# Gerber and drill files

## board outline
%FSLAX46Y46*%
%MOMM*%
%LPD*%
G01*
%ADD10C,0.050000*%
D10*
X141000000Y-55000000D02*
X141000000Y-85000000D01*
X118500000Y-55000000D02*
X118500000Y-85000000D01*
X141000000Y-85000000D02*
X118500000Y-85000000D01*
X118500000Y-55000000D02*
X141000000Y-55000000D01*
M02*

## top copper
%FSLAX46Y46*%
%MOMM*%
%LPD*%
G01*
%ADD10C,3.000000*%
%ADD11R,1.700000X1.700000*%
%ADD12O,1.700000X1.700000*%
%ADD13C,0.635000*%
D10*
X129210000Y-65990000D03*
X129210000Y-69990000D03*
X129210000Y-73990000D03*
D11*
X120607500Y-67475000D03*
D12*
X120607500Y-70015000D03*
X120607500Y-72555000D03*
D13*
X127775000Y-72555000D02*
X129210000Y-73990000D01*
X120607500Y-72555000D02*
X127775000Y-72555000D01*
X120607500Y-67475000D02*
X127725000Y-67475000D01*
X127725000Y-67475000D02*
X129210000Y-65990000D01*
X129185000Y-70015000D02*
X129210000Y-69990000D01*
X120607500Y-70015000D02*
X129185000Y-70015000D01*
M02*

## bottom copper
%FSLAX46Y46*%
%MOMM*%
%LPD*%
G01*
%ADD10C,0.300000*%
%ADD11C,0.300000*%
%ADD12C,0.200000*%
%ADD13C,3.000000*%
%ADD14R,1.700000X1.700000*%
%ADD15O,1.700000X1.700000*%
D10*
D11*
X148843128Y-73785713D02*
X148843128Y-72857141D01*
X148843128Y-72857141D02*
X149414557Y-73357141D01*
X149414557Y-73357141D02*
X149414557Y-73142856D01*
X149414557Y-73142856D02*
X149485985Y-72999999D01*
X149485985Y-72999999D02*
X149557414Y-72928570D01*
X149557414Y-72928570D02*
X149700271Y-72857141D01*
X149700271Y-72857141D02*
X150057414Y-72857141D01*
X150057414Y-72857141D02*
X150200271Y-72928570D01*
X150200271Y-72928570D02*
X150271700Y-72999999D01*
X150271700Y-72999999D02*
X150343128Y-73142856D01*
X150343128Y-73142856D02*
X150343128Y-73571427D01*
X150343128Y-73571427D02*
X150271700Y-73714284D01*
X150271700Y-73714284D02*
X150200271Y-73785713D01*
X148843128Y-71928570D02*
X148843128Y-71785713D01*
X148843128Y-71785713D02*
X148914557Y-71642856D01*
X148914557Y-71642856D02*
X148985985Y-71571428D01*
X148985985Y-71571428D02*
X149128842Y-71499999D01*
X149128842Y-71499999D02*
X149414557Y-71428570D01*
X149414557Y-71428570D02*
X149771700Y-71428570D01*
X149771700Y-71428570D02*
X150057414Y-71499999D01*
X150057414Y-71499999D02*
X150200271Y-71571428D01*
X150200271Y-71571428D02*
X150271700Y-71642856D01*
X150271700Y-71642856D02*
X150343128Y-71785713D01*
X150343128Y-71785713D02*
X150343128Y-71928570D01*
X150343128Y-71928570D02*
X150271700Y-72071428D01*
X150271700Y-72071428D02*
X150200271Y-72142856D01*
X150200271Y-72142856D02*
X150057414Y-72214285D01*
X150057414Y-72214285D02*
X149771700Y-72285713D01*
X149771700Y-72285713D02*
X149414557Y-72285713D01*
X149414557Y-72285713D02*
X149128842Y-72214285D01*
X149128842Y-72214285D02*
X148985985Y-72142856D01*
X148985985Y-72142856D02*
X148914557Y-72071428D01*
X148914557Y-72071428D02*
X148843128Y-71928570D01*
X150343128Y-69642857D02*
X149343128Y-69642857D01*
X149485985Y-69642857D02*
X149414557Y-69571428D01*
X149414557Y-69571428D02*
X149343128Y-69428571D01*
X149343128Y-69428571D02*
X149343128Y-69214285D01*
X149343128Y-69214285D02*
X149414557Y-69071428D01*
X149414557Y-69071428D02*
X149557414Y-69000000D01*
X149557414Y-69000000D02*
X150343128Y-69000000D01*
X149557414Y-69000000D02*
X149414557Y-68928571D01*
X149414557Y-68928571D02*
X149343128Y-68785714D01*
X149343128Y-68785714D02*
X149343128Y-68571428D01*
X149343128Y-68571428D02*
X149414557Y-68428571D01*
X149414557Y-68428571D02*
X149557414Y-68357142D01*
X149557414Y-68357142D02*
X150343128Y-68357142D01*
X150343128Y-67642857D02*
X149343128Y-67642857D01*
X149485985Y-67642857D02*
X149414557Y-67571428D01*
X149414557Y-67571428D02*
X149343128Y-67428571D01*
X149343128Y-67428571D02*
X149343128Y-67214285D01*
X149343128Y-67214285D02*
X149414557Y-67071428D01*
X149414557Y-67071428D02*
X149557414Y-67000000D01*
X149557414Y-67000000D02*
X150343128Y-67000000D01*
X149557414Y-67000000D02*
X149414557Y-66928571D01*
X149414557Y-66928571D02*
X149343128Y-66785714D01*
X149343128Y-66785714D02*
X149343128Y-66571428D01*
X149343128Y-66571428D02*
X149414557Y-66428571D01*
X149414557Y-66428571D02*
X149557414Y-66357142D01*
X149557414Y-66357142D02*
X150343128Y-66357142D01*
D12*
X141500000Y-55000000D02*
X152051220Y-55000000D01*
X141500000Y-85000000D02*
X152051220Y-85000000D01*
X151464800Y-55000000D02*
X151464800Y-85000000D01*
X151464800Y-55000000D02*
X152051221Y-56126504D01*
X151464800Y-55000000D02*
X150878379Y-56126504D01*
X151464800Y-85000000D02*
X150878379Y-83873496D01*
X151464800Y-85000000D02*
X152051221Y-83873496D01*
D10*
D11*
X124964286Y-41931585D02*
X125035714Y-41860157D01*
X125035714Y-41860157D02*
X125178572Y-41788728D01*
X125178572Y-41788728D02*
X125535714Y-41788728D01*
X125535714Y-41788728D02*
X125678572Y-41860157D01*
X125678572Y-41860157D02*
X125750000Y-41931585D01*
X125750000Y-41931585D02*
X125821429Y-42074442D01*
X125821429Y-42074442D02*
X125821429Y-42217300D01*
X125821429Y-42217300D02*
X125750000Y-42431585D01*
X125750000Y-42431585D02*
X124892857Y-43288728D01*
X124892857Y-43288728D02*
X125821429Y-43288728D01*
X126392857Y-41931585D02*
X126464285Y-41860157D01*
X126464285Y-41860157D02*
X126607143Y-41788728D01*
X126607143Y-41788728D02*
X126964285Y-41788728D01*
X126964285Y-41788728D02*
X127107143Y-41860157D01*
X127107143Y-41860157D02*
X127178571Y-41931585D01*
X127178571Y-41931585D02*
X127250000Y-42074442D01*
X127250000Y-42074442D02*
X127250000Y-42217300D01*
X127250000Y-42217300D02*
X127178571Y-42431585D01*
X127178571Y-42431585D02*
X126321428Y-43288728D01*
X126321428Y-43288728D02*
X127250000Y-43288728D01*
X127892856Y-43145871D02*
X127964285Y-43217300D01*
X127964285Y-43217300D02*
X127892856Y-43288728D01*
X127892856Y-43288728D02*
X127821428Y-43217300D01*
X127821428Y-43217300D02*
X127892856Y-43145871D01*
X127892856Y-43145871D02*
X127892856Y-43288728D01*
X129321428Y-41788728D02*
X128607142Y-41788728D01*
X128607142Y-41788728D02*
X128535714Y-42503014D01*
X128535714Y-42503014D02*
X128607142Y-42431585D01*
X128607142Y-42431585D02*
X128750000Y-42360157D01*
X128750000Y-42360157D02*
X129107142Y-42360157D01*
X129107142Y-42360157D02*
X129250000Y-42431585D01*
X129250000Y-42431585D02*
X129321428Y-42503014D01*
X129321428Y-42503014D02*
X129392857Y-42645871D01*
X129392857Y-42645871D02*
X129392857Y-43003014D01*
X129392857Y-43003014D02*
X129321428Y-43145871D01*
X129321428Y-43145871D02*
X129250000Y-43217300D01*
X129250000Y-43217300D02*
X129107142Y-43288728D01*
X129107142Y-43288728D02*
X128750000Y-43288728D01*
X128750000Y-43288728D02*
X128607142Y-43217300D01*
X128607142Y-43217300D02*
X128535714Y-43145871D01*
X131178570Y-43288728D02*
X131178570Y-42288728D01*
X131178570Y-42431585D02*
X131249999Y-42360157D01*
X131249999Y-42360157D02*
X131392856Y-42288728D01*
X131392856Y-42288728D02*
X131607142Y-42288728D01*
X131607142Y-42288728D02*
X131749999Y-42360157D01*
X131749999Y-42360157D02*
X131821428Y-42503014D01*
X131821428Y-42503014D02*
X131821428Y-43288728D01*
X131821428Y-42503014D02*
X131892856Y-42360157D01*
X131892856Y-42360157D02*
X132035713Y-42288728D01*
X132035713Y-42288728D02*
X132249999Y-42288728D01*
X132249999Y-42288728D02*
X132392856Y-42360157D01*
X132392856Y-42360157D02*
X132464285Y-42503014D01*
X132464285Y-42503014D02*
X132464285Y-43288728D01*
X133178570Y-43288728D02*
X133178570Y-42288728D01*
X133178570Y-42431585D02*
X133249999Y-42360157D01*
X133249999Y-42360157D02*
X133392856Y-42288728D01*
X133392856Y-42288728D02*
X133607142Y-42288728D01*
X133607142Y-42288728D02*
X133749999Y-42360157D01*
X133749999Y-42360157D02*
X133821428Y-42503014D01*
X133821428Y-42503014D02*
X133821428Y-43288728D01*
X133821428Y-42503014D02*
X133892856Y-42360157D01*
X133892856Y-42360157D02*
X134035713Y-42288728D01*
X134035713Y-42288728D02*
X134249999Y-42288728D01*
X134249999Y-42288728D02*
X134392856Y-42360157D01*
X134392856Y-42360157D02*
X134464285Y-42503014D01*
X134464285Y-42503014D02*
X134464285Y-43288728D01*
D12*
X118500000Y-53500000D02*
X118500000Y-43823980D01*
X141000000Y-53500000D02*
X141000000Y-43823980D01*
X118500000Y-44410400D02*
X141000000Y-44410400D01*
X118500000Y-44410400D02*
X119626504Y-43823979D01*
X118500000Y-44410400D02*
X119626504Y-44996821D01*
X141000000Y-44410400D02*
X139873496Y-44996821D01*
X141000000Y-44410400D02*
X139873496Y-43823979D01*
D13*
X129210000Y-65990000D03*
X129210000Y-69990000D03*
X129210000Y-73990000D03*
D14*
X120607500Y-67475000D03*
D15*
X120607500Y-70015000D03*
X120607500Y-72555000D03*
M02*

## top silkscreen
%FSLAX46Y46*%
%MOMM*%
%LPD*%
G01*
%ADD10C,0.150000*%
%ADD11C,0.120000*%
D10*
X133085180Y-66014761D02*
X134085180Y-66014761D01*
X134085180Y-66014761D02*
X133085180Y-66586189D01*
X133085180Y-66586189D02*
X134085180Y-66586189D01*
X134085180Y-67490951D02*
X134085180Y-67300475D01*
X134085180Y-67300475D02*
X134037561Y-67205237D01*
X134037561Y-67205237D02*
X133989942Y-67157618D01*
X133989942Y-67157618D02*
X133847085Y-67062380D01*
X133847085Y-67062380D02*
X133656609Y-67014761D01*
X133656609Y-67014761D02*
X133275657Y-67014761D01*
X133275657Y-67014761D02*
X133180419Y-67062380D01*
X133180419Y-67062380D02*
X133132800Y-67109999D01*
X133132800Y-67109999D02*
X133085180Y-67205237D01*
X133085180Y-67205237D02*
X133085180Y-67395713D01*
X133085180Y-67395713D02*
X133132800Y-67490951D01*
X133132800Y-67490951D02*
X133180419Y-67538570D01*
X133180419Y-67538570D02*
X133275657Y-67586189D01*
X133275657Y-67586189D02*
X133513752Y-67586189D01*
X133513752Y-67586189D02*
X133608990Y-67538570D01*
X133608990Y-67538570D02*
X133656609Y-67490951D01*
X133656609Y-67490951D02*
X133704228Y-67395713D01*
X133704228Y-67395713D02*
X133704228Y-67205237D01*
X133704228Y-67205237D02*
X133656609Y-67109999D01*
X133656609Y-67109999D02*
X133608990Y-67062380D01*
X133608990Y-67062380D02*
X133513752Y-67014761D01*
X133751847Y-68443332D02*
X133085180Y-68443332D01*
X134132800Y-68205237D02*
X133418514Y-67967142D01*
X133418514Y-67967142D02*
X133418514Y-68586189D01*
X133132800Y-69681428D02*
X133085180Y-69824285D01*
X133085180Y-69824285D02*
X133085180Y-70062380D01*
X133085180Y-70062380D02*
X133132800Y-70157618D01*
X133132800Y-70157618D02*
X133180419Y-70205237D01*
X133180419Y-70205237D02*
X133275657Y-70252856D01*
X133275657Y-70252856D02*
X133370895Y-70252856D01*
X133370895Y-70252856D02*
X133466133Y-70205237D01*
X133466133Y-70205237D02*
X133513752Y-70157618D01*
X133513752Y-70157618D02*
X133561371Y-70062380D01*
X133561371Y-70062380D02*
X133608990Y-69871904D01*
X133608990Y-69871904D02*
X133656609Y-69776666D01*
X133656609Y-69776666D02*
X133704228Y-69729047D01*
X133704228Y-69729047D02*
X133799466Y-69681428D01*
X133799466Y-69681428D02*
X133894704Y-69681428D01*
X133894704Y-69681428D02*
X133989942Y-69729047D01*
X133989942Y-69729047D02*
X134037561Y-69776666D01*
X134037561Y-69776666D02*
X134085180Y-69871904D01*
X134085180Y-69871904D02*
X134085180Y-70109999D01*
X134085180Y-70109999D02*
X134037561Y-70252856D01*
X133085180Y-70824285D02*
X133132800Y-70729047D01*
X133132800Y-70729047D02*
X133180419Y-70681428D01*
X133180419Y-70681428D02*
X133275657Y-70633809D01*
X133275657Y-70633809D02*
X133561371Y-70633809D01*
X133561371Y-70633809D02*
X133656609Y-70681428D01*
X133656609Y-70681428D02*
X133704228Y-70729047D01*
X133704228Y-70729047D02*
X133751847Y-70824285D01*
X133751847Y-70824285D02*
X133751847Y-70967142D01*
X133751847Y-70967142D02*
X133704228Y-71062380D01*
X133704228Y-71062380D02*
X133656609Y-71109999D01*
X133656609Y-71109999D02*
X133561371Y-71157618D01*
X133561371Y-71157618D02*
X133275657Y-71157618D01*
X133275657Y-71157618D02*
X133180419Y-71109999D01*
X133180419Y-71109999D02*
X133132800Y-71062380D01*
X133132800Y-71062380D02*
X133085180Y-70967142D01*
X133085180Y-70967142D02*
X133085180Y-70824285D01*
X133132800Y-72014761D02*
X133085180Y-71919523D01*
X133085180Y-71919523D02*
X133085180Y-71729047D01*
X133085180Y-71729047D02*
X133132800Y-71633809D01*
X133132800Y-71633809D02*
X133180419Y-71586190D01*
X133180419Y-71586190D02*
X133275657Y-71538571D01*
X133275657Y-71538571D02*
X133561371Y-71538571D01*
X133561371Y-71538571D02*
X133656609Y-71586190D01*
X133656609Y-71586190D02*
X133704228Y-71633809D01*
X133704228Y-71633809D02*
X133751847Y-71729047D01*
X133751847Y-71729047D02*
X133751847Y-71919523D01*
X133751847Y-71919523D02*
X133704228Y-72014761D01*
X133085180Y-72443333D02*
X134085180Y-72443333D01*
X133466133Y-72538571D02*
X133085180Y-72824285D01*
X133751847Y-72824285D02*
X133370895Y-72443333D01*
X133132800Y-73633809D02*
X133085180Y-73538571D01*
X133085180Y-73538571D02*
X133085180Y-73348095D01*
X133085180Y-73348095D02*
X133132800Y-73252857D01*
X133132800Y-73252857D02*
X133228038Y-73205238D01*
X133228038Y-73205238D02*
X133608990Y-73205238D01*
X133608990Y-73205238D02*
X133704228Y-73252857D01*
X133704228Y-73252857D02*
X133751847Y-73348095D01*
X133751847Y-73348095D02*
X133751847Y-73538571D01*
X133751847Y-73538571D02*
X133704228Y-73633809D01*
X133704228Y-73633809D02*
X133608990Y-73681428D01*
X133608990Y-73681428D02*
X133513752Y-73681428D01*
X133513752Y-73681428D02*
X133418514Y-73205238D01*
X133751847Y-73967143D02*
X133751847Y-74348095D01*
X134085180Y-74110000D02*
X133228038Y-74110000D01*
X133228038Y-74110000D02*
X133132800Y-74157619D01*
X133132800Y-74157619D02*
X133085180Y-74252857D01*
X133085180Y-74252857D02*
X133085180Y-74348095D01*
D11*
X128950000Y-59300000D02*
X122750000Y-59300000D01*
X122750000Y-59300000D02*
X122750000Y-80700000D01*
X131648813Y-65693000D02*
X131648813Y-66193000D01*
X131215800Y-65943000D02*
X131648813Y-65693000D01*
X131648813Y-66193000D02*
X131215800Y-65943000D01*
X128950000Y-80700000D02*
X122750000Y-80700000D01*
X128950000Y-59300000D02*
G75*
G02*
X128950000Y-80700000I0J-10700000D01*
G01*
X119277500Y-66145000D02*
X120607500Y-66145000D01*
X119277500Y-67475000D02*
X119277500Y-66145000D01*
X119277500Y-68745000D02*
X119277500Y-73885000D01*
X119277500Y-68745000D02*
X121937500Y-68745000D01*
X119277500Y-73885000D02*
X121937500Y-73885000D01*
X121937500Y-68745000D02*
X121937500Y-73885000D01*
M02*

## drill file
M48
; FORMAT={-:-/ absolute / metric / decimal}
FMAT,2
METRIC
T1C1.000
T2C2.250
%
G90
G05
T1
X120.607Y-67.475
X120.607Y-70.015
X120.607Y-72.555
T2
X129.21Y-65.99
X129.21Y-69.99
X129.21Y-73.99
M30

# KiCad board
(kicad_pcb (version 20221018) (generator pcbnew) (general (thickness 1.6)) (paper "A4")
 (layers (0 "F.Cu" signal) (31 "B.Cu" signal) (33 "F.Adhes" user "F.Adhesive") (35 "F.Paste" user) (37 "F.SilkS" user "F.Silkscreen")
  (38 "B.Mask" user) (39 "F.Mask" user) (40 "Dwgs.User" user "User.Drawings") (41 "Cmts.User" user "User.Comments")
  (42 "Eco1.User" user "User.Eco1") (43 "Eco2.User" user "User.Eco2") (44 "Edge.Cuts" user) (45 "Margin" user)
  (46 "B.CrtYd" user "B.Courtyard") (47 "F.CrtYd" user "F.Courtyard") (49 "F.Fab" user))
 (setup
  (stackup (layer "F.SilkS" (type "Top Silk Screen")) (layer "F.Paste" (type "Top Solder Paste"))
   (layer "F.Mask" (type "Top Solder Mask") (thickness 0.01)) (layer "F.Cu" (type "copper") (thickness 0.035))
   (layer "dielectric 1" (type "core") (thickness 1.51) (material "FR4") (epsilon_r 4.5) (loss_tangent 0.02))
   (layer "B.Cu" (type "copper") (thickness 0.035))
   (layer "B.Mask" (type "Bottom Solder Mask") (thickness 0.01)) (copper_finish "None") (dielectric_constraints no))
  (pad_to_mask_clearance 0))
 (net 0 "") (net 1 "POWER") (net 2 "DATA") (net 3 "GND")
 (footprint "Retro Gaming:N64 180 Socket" (layer "F.Cu") (at 129.26 69.88 -90)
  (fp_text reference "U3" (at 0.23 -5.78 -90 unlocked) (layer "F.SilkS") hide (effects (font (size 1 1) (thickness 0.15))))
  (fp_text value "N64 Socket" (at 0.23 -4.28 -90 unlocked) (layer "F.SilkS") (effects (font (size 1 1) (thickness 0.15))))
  (fp_line (start -10.58 0.31) (end -10.58 6.51) (stroke (width 0.12) (type solid)) (layer "F.SilkS"))
  (fp_line (start -10.58 6.51) (end 10.82 6.51) (stroke (width 0.12) (type solid)) (layer "F.SilkS"))
  (fp_line (start -4.187 -2.388813) (end -3.687 -2.388813) (stroke (width 0.12) (type solid)) (layer "F.SilkS"))
  (fp_line (start -3.937 -1.9558) (end -4.187 -2.388813) (stroke (width 0.12) (type solid)) (layer "F.SilkS"))
  (fp_line (start -3.687 -2.388813) (end -3.937 -1.9558) (stroke (width 0.12) (type solid)) (layer "F.SilkS"))
  (fp_line (start 10.82 0.31) (end 10.82 6.51) (stroke (width 0.12) (type solid)) (layer "F.SilkS"))
  (fp_arc (start -10.58 0.31) (mid 0.12 -10.39) (end 10.82 0.31) (stroke (width 0.12) (type solid)) (layer "F.SilkS"))
  (pad "1" thru_hole circle (at -3.89 0.05 270) (size 3 3) (drill 2.25) (layers "*.Cu" "*.Mask") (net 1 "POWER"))
  (pad "2" thru_hole circle (at 0.11 0.05 270) (size 3 3) (drill 2.25) (layers "*.Cu" "*.Mask") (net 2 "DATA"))
  (pad "3" thru_hole circle (at 4.11 0.05 270) (size 3 3) (drill 2.25) (layers "*.Cu" "*.Mask") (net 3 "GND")))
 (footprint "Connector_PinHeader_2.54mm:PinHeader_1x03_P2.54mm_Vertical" (layer "F.Cu") (at 120.6075 67.475)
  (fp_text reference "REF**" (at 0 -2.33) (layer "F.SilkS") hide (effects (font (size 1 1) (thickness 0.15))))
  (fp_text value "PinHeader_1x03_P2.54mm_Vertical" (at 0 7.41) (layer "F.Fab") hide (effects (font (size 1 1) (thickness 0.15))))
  (fp_line (start -1.33 -1.33) (end 0 -1.33) (stroke (width 0.12) (type solid)) (layer "F.SilkS"))
  (fp_line (start -1.33 0) (end -1.33 -1.33) (stroke (width 0.12) (type solid)) (layer "F.SilkS"))
  (fp_line (start -1.33 1.27) (end -1.33 6.41) (stroke (width 0.12) (type solid)) (layer "F.SilkS"))
  (fp_line (start -1.33 1.27) (end 1.33 1.27) (stroke (width 0.12) (type solid)) (layer "F.SilkS"))
  (fp_line (start -1.33 6.41) (end 1.33 6.41) (stroke (width 0.12) (type solid)) (layer "F.SilkS"))
  (fp_line (start 1.33 1.27) (end 1.33 6.41) (stroke (width 0.12) (type solid)) (layer "F.SilkS"))
  (pad "1" thru_hole rect (at 0 0) (size 1.7 1.7) (drill 1) (layers "*.Cu" "*.Mask") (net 1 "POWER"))
  (pad "2" thru_hole oval (at 0 2.54) (size 1.7 1.7) (drill 1) (layers "*.Cu" "*.Mask") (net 2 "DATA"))
  (pad "3" thru_hole oval (at 0 5.08) (size 1.7 1.7) (drill 1) (layers "*.Cu" "*.Mask") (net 3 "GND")))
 (gr_line (start 141 55) (end 141 85) (stroke (width 0.05) (type solid)) (layer "Edge.Cuts"))
 (gr_line (start 118.5 55) (end 118.5 85) (stroke (width 0.05) (type solid)) (layer "Edge.Cuts"))
 (gr_line (start 141 85) (end 118.5 85) (stroke (width 0.05) (type solid)) (layer "Edge.Cuts"))
 (gr_line (start 118.5 55) (end 141 55) (stroke (width 0.05) (type solid)) (layer "Edge.Cuts"))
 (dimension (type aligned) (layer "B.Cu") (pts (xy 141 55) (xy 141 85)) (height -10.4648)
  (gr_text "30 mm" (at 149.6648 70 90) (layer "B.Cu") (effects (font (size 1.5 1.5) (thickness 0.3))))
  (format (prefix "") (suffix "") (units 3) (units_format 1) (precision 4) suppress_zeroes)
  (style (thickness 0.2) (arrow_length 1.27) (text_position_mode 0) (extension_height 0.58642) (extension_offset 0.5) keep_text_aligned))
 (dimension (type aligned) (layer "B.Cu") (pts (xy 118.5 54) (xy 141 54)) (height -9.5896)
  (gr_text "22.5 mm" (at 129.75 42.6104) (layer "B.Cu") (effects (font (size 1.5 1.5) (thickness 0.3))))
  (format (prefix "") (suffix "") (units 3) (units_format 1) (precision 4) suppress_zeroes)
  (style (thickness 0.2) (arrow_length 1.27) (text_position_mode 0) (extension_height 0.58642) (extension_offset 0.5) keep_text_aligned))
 (segment (start 127.775 72.555) (end 129.21 73.99) (width 0.635) (layer "F.Cu") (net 3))
 (segment (start 120.6075 72.555) (end 127.775 72.555) (width 0.635) (layer "F.Cu") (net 3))
 (segment (start 120.6075 67.475) (end 127.725 67.475) (width 0.635) (layer "F.Cu") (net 1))
 (segment (start 127.725 67.475) (end 129.21 65.99) (width 0.635) (layer "F.Cu") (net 1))
 (segment (start 129.185 70.015) (end 129.21 69.99) (width 0.635) (layer "F.Cu") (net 2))
 (segment (start 120.6075 70.015) (end 129.185 70.015) (width 0.635) (layer "F.Cu") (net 2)))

